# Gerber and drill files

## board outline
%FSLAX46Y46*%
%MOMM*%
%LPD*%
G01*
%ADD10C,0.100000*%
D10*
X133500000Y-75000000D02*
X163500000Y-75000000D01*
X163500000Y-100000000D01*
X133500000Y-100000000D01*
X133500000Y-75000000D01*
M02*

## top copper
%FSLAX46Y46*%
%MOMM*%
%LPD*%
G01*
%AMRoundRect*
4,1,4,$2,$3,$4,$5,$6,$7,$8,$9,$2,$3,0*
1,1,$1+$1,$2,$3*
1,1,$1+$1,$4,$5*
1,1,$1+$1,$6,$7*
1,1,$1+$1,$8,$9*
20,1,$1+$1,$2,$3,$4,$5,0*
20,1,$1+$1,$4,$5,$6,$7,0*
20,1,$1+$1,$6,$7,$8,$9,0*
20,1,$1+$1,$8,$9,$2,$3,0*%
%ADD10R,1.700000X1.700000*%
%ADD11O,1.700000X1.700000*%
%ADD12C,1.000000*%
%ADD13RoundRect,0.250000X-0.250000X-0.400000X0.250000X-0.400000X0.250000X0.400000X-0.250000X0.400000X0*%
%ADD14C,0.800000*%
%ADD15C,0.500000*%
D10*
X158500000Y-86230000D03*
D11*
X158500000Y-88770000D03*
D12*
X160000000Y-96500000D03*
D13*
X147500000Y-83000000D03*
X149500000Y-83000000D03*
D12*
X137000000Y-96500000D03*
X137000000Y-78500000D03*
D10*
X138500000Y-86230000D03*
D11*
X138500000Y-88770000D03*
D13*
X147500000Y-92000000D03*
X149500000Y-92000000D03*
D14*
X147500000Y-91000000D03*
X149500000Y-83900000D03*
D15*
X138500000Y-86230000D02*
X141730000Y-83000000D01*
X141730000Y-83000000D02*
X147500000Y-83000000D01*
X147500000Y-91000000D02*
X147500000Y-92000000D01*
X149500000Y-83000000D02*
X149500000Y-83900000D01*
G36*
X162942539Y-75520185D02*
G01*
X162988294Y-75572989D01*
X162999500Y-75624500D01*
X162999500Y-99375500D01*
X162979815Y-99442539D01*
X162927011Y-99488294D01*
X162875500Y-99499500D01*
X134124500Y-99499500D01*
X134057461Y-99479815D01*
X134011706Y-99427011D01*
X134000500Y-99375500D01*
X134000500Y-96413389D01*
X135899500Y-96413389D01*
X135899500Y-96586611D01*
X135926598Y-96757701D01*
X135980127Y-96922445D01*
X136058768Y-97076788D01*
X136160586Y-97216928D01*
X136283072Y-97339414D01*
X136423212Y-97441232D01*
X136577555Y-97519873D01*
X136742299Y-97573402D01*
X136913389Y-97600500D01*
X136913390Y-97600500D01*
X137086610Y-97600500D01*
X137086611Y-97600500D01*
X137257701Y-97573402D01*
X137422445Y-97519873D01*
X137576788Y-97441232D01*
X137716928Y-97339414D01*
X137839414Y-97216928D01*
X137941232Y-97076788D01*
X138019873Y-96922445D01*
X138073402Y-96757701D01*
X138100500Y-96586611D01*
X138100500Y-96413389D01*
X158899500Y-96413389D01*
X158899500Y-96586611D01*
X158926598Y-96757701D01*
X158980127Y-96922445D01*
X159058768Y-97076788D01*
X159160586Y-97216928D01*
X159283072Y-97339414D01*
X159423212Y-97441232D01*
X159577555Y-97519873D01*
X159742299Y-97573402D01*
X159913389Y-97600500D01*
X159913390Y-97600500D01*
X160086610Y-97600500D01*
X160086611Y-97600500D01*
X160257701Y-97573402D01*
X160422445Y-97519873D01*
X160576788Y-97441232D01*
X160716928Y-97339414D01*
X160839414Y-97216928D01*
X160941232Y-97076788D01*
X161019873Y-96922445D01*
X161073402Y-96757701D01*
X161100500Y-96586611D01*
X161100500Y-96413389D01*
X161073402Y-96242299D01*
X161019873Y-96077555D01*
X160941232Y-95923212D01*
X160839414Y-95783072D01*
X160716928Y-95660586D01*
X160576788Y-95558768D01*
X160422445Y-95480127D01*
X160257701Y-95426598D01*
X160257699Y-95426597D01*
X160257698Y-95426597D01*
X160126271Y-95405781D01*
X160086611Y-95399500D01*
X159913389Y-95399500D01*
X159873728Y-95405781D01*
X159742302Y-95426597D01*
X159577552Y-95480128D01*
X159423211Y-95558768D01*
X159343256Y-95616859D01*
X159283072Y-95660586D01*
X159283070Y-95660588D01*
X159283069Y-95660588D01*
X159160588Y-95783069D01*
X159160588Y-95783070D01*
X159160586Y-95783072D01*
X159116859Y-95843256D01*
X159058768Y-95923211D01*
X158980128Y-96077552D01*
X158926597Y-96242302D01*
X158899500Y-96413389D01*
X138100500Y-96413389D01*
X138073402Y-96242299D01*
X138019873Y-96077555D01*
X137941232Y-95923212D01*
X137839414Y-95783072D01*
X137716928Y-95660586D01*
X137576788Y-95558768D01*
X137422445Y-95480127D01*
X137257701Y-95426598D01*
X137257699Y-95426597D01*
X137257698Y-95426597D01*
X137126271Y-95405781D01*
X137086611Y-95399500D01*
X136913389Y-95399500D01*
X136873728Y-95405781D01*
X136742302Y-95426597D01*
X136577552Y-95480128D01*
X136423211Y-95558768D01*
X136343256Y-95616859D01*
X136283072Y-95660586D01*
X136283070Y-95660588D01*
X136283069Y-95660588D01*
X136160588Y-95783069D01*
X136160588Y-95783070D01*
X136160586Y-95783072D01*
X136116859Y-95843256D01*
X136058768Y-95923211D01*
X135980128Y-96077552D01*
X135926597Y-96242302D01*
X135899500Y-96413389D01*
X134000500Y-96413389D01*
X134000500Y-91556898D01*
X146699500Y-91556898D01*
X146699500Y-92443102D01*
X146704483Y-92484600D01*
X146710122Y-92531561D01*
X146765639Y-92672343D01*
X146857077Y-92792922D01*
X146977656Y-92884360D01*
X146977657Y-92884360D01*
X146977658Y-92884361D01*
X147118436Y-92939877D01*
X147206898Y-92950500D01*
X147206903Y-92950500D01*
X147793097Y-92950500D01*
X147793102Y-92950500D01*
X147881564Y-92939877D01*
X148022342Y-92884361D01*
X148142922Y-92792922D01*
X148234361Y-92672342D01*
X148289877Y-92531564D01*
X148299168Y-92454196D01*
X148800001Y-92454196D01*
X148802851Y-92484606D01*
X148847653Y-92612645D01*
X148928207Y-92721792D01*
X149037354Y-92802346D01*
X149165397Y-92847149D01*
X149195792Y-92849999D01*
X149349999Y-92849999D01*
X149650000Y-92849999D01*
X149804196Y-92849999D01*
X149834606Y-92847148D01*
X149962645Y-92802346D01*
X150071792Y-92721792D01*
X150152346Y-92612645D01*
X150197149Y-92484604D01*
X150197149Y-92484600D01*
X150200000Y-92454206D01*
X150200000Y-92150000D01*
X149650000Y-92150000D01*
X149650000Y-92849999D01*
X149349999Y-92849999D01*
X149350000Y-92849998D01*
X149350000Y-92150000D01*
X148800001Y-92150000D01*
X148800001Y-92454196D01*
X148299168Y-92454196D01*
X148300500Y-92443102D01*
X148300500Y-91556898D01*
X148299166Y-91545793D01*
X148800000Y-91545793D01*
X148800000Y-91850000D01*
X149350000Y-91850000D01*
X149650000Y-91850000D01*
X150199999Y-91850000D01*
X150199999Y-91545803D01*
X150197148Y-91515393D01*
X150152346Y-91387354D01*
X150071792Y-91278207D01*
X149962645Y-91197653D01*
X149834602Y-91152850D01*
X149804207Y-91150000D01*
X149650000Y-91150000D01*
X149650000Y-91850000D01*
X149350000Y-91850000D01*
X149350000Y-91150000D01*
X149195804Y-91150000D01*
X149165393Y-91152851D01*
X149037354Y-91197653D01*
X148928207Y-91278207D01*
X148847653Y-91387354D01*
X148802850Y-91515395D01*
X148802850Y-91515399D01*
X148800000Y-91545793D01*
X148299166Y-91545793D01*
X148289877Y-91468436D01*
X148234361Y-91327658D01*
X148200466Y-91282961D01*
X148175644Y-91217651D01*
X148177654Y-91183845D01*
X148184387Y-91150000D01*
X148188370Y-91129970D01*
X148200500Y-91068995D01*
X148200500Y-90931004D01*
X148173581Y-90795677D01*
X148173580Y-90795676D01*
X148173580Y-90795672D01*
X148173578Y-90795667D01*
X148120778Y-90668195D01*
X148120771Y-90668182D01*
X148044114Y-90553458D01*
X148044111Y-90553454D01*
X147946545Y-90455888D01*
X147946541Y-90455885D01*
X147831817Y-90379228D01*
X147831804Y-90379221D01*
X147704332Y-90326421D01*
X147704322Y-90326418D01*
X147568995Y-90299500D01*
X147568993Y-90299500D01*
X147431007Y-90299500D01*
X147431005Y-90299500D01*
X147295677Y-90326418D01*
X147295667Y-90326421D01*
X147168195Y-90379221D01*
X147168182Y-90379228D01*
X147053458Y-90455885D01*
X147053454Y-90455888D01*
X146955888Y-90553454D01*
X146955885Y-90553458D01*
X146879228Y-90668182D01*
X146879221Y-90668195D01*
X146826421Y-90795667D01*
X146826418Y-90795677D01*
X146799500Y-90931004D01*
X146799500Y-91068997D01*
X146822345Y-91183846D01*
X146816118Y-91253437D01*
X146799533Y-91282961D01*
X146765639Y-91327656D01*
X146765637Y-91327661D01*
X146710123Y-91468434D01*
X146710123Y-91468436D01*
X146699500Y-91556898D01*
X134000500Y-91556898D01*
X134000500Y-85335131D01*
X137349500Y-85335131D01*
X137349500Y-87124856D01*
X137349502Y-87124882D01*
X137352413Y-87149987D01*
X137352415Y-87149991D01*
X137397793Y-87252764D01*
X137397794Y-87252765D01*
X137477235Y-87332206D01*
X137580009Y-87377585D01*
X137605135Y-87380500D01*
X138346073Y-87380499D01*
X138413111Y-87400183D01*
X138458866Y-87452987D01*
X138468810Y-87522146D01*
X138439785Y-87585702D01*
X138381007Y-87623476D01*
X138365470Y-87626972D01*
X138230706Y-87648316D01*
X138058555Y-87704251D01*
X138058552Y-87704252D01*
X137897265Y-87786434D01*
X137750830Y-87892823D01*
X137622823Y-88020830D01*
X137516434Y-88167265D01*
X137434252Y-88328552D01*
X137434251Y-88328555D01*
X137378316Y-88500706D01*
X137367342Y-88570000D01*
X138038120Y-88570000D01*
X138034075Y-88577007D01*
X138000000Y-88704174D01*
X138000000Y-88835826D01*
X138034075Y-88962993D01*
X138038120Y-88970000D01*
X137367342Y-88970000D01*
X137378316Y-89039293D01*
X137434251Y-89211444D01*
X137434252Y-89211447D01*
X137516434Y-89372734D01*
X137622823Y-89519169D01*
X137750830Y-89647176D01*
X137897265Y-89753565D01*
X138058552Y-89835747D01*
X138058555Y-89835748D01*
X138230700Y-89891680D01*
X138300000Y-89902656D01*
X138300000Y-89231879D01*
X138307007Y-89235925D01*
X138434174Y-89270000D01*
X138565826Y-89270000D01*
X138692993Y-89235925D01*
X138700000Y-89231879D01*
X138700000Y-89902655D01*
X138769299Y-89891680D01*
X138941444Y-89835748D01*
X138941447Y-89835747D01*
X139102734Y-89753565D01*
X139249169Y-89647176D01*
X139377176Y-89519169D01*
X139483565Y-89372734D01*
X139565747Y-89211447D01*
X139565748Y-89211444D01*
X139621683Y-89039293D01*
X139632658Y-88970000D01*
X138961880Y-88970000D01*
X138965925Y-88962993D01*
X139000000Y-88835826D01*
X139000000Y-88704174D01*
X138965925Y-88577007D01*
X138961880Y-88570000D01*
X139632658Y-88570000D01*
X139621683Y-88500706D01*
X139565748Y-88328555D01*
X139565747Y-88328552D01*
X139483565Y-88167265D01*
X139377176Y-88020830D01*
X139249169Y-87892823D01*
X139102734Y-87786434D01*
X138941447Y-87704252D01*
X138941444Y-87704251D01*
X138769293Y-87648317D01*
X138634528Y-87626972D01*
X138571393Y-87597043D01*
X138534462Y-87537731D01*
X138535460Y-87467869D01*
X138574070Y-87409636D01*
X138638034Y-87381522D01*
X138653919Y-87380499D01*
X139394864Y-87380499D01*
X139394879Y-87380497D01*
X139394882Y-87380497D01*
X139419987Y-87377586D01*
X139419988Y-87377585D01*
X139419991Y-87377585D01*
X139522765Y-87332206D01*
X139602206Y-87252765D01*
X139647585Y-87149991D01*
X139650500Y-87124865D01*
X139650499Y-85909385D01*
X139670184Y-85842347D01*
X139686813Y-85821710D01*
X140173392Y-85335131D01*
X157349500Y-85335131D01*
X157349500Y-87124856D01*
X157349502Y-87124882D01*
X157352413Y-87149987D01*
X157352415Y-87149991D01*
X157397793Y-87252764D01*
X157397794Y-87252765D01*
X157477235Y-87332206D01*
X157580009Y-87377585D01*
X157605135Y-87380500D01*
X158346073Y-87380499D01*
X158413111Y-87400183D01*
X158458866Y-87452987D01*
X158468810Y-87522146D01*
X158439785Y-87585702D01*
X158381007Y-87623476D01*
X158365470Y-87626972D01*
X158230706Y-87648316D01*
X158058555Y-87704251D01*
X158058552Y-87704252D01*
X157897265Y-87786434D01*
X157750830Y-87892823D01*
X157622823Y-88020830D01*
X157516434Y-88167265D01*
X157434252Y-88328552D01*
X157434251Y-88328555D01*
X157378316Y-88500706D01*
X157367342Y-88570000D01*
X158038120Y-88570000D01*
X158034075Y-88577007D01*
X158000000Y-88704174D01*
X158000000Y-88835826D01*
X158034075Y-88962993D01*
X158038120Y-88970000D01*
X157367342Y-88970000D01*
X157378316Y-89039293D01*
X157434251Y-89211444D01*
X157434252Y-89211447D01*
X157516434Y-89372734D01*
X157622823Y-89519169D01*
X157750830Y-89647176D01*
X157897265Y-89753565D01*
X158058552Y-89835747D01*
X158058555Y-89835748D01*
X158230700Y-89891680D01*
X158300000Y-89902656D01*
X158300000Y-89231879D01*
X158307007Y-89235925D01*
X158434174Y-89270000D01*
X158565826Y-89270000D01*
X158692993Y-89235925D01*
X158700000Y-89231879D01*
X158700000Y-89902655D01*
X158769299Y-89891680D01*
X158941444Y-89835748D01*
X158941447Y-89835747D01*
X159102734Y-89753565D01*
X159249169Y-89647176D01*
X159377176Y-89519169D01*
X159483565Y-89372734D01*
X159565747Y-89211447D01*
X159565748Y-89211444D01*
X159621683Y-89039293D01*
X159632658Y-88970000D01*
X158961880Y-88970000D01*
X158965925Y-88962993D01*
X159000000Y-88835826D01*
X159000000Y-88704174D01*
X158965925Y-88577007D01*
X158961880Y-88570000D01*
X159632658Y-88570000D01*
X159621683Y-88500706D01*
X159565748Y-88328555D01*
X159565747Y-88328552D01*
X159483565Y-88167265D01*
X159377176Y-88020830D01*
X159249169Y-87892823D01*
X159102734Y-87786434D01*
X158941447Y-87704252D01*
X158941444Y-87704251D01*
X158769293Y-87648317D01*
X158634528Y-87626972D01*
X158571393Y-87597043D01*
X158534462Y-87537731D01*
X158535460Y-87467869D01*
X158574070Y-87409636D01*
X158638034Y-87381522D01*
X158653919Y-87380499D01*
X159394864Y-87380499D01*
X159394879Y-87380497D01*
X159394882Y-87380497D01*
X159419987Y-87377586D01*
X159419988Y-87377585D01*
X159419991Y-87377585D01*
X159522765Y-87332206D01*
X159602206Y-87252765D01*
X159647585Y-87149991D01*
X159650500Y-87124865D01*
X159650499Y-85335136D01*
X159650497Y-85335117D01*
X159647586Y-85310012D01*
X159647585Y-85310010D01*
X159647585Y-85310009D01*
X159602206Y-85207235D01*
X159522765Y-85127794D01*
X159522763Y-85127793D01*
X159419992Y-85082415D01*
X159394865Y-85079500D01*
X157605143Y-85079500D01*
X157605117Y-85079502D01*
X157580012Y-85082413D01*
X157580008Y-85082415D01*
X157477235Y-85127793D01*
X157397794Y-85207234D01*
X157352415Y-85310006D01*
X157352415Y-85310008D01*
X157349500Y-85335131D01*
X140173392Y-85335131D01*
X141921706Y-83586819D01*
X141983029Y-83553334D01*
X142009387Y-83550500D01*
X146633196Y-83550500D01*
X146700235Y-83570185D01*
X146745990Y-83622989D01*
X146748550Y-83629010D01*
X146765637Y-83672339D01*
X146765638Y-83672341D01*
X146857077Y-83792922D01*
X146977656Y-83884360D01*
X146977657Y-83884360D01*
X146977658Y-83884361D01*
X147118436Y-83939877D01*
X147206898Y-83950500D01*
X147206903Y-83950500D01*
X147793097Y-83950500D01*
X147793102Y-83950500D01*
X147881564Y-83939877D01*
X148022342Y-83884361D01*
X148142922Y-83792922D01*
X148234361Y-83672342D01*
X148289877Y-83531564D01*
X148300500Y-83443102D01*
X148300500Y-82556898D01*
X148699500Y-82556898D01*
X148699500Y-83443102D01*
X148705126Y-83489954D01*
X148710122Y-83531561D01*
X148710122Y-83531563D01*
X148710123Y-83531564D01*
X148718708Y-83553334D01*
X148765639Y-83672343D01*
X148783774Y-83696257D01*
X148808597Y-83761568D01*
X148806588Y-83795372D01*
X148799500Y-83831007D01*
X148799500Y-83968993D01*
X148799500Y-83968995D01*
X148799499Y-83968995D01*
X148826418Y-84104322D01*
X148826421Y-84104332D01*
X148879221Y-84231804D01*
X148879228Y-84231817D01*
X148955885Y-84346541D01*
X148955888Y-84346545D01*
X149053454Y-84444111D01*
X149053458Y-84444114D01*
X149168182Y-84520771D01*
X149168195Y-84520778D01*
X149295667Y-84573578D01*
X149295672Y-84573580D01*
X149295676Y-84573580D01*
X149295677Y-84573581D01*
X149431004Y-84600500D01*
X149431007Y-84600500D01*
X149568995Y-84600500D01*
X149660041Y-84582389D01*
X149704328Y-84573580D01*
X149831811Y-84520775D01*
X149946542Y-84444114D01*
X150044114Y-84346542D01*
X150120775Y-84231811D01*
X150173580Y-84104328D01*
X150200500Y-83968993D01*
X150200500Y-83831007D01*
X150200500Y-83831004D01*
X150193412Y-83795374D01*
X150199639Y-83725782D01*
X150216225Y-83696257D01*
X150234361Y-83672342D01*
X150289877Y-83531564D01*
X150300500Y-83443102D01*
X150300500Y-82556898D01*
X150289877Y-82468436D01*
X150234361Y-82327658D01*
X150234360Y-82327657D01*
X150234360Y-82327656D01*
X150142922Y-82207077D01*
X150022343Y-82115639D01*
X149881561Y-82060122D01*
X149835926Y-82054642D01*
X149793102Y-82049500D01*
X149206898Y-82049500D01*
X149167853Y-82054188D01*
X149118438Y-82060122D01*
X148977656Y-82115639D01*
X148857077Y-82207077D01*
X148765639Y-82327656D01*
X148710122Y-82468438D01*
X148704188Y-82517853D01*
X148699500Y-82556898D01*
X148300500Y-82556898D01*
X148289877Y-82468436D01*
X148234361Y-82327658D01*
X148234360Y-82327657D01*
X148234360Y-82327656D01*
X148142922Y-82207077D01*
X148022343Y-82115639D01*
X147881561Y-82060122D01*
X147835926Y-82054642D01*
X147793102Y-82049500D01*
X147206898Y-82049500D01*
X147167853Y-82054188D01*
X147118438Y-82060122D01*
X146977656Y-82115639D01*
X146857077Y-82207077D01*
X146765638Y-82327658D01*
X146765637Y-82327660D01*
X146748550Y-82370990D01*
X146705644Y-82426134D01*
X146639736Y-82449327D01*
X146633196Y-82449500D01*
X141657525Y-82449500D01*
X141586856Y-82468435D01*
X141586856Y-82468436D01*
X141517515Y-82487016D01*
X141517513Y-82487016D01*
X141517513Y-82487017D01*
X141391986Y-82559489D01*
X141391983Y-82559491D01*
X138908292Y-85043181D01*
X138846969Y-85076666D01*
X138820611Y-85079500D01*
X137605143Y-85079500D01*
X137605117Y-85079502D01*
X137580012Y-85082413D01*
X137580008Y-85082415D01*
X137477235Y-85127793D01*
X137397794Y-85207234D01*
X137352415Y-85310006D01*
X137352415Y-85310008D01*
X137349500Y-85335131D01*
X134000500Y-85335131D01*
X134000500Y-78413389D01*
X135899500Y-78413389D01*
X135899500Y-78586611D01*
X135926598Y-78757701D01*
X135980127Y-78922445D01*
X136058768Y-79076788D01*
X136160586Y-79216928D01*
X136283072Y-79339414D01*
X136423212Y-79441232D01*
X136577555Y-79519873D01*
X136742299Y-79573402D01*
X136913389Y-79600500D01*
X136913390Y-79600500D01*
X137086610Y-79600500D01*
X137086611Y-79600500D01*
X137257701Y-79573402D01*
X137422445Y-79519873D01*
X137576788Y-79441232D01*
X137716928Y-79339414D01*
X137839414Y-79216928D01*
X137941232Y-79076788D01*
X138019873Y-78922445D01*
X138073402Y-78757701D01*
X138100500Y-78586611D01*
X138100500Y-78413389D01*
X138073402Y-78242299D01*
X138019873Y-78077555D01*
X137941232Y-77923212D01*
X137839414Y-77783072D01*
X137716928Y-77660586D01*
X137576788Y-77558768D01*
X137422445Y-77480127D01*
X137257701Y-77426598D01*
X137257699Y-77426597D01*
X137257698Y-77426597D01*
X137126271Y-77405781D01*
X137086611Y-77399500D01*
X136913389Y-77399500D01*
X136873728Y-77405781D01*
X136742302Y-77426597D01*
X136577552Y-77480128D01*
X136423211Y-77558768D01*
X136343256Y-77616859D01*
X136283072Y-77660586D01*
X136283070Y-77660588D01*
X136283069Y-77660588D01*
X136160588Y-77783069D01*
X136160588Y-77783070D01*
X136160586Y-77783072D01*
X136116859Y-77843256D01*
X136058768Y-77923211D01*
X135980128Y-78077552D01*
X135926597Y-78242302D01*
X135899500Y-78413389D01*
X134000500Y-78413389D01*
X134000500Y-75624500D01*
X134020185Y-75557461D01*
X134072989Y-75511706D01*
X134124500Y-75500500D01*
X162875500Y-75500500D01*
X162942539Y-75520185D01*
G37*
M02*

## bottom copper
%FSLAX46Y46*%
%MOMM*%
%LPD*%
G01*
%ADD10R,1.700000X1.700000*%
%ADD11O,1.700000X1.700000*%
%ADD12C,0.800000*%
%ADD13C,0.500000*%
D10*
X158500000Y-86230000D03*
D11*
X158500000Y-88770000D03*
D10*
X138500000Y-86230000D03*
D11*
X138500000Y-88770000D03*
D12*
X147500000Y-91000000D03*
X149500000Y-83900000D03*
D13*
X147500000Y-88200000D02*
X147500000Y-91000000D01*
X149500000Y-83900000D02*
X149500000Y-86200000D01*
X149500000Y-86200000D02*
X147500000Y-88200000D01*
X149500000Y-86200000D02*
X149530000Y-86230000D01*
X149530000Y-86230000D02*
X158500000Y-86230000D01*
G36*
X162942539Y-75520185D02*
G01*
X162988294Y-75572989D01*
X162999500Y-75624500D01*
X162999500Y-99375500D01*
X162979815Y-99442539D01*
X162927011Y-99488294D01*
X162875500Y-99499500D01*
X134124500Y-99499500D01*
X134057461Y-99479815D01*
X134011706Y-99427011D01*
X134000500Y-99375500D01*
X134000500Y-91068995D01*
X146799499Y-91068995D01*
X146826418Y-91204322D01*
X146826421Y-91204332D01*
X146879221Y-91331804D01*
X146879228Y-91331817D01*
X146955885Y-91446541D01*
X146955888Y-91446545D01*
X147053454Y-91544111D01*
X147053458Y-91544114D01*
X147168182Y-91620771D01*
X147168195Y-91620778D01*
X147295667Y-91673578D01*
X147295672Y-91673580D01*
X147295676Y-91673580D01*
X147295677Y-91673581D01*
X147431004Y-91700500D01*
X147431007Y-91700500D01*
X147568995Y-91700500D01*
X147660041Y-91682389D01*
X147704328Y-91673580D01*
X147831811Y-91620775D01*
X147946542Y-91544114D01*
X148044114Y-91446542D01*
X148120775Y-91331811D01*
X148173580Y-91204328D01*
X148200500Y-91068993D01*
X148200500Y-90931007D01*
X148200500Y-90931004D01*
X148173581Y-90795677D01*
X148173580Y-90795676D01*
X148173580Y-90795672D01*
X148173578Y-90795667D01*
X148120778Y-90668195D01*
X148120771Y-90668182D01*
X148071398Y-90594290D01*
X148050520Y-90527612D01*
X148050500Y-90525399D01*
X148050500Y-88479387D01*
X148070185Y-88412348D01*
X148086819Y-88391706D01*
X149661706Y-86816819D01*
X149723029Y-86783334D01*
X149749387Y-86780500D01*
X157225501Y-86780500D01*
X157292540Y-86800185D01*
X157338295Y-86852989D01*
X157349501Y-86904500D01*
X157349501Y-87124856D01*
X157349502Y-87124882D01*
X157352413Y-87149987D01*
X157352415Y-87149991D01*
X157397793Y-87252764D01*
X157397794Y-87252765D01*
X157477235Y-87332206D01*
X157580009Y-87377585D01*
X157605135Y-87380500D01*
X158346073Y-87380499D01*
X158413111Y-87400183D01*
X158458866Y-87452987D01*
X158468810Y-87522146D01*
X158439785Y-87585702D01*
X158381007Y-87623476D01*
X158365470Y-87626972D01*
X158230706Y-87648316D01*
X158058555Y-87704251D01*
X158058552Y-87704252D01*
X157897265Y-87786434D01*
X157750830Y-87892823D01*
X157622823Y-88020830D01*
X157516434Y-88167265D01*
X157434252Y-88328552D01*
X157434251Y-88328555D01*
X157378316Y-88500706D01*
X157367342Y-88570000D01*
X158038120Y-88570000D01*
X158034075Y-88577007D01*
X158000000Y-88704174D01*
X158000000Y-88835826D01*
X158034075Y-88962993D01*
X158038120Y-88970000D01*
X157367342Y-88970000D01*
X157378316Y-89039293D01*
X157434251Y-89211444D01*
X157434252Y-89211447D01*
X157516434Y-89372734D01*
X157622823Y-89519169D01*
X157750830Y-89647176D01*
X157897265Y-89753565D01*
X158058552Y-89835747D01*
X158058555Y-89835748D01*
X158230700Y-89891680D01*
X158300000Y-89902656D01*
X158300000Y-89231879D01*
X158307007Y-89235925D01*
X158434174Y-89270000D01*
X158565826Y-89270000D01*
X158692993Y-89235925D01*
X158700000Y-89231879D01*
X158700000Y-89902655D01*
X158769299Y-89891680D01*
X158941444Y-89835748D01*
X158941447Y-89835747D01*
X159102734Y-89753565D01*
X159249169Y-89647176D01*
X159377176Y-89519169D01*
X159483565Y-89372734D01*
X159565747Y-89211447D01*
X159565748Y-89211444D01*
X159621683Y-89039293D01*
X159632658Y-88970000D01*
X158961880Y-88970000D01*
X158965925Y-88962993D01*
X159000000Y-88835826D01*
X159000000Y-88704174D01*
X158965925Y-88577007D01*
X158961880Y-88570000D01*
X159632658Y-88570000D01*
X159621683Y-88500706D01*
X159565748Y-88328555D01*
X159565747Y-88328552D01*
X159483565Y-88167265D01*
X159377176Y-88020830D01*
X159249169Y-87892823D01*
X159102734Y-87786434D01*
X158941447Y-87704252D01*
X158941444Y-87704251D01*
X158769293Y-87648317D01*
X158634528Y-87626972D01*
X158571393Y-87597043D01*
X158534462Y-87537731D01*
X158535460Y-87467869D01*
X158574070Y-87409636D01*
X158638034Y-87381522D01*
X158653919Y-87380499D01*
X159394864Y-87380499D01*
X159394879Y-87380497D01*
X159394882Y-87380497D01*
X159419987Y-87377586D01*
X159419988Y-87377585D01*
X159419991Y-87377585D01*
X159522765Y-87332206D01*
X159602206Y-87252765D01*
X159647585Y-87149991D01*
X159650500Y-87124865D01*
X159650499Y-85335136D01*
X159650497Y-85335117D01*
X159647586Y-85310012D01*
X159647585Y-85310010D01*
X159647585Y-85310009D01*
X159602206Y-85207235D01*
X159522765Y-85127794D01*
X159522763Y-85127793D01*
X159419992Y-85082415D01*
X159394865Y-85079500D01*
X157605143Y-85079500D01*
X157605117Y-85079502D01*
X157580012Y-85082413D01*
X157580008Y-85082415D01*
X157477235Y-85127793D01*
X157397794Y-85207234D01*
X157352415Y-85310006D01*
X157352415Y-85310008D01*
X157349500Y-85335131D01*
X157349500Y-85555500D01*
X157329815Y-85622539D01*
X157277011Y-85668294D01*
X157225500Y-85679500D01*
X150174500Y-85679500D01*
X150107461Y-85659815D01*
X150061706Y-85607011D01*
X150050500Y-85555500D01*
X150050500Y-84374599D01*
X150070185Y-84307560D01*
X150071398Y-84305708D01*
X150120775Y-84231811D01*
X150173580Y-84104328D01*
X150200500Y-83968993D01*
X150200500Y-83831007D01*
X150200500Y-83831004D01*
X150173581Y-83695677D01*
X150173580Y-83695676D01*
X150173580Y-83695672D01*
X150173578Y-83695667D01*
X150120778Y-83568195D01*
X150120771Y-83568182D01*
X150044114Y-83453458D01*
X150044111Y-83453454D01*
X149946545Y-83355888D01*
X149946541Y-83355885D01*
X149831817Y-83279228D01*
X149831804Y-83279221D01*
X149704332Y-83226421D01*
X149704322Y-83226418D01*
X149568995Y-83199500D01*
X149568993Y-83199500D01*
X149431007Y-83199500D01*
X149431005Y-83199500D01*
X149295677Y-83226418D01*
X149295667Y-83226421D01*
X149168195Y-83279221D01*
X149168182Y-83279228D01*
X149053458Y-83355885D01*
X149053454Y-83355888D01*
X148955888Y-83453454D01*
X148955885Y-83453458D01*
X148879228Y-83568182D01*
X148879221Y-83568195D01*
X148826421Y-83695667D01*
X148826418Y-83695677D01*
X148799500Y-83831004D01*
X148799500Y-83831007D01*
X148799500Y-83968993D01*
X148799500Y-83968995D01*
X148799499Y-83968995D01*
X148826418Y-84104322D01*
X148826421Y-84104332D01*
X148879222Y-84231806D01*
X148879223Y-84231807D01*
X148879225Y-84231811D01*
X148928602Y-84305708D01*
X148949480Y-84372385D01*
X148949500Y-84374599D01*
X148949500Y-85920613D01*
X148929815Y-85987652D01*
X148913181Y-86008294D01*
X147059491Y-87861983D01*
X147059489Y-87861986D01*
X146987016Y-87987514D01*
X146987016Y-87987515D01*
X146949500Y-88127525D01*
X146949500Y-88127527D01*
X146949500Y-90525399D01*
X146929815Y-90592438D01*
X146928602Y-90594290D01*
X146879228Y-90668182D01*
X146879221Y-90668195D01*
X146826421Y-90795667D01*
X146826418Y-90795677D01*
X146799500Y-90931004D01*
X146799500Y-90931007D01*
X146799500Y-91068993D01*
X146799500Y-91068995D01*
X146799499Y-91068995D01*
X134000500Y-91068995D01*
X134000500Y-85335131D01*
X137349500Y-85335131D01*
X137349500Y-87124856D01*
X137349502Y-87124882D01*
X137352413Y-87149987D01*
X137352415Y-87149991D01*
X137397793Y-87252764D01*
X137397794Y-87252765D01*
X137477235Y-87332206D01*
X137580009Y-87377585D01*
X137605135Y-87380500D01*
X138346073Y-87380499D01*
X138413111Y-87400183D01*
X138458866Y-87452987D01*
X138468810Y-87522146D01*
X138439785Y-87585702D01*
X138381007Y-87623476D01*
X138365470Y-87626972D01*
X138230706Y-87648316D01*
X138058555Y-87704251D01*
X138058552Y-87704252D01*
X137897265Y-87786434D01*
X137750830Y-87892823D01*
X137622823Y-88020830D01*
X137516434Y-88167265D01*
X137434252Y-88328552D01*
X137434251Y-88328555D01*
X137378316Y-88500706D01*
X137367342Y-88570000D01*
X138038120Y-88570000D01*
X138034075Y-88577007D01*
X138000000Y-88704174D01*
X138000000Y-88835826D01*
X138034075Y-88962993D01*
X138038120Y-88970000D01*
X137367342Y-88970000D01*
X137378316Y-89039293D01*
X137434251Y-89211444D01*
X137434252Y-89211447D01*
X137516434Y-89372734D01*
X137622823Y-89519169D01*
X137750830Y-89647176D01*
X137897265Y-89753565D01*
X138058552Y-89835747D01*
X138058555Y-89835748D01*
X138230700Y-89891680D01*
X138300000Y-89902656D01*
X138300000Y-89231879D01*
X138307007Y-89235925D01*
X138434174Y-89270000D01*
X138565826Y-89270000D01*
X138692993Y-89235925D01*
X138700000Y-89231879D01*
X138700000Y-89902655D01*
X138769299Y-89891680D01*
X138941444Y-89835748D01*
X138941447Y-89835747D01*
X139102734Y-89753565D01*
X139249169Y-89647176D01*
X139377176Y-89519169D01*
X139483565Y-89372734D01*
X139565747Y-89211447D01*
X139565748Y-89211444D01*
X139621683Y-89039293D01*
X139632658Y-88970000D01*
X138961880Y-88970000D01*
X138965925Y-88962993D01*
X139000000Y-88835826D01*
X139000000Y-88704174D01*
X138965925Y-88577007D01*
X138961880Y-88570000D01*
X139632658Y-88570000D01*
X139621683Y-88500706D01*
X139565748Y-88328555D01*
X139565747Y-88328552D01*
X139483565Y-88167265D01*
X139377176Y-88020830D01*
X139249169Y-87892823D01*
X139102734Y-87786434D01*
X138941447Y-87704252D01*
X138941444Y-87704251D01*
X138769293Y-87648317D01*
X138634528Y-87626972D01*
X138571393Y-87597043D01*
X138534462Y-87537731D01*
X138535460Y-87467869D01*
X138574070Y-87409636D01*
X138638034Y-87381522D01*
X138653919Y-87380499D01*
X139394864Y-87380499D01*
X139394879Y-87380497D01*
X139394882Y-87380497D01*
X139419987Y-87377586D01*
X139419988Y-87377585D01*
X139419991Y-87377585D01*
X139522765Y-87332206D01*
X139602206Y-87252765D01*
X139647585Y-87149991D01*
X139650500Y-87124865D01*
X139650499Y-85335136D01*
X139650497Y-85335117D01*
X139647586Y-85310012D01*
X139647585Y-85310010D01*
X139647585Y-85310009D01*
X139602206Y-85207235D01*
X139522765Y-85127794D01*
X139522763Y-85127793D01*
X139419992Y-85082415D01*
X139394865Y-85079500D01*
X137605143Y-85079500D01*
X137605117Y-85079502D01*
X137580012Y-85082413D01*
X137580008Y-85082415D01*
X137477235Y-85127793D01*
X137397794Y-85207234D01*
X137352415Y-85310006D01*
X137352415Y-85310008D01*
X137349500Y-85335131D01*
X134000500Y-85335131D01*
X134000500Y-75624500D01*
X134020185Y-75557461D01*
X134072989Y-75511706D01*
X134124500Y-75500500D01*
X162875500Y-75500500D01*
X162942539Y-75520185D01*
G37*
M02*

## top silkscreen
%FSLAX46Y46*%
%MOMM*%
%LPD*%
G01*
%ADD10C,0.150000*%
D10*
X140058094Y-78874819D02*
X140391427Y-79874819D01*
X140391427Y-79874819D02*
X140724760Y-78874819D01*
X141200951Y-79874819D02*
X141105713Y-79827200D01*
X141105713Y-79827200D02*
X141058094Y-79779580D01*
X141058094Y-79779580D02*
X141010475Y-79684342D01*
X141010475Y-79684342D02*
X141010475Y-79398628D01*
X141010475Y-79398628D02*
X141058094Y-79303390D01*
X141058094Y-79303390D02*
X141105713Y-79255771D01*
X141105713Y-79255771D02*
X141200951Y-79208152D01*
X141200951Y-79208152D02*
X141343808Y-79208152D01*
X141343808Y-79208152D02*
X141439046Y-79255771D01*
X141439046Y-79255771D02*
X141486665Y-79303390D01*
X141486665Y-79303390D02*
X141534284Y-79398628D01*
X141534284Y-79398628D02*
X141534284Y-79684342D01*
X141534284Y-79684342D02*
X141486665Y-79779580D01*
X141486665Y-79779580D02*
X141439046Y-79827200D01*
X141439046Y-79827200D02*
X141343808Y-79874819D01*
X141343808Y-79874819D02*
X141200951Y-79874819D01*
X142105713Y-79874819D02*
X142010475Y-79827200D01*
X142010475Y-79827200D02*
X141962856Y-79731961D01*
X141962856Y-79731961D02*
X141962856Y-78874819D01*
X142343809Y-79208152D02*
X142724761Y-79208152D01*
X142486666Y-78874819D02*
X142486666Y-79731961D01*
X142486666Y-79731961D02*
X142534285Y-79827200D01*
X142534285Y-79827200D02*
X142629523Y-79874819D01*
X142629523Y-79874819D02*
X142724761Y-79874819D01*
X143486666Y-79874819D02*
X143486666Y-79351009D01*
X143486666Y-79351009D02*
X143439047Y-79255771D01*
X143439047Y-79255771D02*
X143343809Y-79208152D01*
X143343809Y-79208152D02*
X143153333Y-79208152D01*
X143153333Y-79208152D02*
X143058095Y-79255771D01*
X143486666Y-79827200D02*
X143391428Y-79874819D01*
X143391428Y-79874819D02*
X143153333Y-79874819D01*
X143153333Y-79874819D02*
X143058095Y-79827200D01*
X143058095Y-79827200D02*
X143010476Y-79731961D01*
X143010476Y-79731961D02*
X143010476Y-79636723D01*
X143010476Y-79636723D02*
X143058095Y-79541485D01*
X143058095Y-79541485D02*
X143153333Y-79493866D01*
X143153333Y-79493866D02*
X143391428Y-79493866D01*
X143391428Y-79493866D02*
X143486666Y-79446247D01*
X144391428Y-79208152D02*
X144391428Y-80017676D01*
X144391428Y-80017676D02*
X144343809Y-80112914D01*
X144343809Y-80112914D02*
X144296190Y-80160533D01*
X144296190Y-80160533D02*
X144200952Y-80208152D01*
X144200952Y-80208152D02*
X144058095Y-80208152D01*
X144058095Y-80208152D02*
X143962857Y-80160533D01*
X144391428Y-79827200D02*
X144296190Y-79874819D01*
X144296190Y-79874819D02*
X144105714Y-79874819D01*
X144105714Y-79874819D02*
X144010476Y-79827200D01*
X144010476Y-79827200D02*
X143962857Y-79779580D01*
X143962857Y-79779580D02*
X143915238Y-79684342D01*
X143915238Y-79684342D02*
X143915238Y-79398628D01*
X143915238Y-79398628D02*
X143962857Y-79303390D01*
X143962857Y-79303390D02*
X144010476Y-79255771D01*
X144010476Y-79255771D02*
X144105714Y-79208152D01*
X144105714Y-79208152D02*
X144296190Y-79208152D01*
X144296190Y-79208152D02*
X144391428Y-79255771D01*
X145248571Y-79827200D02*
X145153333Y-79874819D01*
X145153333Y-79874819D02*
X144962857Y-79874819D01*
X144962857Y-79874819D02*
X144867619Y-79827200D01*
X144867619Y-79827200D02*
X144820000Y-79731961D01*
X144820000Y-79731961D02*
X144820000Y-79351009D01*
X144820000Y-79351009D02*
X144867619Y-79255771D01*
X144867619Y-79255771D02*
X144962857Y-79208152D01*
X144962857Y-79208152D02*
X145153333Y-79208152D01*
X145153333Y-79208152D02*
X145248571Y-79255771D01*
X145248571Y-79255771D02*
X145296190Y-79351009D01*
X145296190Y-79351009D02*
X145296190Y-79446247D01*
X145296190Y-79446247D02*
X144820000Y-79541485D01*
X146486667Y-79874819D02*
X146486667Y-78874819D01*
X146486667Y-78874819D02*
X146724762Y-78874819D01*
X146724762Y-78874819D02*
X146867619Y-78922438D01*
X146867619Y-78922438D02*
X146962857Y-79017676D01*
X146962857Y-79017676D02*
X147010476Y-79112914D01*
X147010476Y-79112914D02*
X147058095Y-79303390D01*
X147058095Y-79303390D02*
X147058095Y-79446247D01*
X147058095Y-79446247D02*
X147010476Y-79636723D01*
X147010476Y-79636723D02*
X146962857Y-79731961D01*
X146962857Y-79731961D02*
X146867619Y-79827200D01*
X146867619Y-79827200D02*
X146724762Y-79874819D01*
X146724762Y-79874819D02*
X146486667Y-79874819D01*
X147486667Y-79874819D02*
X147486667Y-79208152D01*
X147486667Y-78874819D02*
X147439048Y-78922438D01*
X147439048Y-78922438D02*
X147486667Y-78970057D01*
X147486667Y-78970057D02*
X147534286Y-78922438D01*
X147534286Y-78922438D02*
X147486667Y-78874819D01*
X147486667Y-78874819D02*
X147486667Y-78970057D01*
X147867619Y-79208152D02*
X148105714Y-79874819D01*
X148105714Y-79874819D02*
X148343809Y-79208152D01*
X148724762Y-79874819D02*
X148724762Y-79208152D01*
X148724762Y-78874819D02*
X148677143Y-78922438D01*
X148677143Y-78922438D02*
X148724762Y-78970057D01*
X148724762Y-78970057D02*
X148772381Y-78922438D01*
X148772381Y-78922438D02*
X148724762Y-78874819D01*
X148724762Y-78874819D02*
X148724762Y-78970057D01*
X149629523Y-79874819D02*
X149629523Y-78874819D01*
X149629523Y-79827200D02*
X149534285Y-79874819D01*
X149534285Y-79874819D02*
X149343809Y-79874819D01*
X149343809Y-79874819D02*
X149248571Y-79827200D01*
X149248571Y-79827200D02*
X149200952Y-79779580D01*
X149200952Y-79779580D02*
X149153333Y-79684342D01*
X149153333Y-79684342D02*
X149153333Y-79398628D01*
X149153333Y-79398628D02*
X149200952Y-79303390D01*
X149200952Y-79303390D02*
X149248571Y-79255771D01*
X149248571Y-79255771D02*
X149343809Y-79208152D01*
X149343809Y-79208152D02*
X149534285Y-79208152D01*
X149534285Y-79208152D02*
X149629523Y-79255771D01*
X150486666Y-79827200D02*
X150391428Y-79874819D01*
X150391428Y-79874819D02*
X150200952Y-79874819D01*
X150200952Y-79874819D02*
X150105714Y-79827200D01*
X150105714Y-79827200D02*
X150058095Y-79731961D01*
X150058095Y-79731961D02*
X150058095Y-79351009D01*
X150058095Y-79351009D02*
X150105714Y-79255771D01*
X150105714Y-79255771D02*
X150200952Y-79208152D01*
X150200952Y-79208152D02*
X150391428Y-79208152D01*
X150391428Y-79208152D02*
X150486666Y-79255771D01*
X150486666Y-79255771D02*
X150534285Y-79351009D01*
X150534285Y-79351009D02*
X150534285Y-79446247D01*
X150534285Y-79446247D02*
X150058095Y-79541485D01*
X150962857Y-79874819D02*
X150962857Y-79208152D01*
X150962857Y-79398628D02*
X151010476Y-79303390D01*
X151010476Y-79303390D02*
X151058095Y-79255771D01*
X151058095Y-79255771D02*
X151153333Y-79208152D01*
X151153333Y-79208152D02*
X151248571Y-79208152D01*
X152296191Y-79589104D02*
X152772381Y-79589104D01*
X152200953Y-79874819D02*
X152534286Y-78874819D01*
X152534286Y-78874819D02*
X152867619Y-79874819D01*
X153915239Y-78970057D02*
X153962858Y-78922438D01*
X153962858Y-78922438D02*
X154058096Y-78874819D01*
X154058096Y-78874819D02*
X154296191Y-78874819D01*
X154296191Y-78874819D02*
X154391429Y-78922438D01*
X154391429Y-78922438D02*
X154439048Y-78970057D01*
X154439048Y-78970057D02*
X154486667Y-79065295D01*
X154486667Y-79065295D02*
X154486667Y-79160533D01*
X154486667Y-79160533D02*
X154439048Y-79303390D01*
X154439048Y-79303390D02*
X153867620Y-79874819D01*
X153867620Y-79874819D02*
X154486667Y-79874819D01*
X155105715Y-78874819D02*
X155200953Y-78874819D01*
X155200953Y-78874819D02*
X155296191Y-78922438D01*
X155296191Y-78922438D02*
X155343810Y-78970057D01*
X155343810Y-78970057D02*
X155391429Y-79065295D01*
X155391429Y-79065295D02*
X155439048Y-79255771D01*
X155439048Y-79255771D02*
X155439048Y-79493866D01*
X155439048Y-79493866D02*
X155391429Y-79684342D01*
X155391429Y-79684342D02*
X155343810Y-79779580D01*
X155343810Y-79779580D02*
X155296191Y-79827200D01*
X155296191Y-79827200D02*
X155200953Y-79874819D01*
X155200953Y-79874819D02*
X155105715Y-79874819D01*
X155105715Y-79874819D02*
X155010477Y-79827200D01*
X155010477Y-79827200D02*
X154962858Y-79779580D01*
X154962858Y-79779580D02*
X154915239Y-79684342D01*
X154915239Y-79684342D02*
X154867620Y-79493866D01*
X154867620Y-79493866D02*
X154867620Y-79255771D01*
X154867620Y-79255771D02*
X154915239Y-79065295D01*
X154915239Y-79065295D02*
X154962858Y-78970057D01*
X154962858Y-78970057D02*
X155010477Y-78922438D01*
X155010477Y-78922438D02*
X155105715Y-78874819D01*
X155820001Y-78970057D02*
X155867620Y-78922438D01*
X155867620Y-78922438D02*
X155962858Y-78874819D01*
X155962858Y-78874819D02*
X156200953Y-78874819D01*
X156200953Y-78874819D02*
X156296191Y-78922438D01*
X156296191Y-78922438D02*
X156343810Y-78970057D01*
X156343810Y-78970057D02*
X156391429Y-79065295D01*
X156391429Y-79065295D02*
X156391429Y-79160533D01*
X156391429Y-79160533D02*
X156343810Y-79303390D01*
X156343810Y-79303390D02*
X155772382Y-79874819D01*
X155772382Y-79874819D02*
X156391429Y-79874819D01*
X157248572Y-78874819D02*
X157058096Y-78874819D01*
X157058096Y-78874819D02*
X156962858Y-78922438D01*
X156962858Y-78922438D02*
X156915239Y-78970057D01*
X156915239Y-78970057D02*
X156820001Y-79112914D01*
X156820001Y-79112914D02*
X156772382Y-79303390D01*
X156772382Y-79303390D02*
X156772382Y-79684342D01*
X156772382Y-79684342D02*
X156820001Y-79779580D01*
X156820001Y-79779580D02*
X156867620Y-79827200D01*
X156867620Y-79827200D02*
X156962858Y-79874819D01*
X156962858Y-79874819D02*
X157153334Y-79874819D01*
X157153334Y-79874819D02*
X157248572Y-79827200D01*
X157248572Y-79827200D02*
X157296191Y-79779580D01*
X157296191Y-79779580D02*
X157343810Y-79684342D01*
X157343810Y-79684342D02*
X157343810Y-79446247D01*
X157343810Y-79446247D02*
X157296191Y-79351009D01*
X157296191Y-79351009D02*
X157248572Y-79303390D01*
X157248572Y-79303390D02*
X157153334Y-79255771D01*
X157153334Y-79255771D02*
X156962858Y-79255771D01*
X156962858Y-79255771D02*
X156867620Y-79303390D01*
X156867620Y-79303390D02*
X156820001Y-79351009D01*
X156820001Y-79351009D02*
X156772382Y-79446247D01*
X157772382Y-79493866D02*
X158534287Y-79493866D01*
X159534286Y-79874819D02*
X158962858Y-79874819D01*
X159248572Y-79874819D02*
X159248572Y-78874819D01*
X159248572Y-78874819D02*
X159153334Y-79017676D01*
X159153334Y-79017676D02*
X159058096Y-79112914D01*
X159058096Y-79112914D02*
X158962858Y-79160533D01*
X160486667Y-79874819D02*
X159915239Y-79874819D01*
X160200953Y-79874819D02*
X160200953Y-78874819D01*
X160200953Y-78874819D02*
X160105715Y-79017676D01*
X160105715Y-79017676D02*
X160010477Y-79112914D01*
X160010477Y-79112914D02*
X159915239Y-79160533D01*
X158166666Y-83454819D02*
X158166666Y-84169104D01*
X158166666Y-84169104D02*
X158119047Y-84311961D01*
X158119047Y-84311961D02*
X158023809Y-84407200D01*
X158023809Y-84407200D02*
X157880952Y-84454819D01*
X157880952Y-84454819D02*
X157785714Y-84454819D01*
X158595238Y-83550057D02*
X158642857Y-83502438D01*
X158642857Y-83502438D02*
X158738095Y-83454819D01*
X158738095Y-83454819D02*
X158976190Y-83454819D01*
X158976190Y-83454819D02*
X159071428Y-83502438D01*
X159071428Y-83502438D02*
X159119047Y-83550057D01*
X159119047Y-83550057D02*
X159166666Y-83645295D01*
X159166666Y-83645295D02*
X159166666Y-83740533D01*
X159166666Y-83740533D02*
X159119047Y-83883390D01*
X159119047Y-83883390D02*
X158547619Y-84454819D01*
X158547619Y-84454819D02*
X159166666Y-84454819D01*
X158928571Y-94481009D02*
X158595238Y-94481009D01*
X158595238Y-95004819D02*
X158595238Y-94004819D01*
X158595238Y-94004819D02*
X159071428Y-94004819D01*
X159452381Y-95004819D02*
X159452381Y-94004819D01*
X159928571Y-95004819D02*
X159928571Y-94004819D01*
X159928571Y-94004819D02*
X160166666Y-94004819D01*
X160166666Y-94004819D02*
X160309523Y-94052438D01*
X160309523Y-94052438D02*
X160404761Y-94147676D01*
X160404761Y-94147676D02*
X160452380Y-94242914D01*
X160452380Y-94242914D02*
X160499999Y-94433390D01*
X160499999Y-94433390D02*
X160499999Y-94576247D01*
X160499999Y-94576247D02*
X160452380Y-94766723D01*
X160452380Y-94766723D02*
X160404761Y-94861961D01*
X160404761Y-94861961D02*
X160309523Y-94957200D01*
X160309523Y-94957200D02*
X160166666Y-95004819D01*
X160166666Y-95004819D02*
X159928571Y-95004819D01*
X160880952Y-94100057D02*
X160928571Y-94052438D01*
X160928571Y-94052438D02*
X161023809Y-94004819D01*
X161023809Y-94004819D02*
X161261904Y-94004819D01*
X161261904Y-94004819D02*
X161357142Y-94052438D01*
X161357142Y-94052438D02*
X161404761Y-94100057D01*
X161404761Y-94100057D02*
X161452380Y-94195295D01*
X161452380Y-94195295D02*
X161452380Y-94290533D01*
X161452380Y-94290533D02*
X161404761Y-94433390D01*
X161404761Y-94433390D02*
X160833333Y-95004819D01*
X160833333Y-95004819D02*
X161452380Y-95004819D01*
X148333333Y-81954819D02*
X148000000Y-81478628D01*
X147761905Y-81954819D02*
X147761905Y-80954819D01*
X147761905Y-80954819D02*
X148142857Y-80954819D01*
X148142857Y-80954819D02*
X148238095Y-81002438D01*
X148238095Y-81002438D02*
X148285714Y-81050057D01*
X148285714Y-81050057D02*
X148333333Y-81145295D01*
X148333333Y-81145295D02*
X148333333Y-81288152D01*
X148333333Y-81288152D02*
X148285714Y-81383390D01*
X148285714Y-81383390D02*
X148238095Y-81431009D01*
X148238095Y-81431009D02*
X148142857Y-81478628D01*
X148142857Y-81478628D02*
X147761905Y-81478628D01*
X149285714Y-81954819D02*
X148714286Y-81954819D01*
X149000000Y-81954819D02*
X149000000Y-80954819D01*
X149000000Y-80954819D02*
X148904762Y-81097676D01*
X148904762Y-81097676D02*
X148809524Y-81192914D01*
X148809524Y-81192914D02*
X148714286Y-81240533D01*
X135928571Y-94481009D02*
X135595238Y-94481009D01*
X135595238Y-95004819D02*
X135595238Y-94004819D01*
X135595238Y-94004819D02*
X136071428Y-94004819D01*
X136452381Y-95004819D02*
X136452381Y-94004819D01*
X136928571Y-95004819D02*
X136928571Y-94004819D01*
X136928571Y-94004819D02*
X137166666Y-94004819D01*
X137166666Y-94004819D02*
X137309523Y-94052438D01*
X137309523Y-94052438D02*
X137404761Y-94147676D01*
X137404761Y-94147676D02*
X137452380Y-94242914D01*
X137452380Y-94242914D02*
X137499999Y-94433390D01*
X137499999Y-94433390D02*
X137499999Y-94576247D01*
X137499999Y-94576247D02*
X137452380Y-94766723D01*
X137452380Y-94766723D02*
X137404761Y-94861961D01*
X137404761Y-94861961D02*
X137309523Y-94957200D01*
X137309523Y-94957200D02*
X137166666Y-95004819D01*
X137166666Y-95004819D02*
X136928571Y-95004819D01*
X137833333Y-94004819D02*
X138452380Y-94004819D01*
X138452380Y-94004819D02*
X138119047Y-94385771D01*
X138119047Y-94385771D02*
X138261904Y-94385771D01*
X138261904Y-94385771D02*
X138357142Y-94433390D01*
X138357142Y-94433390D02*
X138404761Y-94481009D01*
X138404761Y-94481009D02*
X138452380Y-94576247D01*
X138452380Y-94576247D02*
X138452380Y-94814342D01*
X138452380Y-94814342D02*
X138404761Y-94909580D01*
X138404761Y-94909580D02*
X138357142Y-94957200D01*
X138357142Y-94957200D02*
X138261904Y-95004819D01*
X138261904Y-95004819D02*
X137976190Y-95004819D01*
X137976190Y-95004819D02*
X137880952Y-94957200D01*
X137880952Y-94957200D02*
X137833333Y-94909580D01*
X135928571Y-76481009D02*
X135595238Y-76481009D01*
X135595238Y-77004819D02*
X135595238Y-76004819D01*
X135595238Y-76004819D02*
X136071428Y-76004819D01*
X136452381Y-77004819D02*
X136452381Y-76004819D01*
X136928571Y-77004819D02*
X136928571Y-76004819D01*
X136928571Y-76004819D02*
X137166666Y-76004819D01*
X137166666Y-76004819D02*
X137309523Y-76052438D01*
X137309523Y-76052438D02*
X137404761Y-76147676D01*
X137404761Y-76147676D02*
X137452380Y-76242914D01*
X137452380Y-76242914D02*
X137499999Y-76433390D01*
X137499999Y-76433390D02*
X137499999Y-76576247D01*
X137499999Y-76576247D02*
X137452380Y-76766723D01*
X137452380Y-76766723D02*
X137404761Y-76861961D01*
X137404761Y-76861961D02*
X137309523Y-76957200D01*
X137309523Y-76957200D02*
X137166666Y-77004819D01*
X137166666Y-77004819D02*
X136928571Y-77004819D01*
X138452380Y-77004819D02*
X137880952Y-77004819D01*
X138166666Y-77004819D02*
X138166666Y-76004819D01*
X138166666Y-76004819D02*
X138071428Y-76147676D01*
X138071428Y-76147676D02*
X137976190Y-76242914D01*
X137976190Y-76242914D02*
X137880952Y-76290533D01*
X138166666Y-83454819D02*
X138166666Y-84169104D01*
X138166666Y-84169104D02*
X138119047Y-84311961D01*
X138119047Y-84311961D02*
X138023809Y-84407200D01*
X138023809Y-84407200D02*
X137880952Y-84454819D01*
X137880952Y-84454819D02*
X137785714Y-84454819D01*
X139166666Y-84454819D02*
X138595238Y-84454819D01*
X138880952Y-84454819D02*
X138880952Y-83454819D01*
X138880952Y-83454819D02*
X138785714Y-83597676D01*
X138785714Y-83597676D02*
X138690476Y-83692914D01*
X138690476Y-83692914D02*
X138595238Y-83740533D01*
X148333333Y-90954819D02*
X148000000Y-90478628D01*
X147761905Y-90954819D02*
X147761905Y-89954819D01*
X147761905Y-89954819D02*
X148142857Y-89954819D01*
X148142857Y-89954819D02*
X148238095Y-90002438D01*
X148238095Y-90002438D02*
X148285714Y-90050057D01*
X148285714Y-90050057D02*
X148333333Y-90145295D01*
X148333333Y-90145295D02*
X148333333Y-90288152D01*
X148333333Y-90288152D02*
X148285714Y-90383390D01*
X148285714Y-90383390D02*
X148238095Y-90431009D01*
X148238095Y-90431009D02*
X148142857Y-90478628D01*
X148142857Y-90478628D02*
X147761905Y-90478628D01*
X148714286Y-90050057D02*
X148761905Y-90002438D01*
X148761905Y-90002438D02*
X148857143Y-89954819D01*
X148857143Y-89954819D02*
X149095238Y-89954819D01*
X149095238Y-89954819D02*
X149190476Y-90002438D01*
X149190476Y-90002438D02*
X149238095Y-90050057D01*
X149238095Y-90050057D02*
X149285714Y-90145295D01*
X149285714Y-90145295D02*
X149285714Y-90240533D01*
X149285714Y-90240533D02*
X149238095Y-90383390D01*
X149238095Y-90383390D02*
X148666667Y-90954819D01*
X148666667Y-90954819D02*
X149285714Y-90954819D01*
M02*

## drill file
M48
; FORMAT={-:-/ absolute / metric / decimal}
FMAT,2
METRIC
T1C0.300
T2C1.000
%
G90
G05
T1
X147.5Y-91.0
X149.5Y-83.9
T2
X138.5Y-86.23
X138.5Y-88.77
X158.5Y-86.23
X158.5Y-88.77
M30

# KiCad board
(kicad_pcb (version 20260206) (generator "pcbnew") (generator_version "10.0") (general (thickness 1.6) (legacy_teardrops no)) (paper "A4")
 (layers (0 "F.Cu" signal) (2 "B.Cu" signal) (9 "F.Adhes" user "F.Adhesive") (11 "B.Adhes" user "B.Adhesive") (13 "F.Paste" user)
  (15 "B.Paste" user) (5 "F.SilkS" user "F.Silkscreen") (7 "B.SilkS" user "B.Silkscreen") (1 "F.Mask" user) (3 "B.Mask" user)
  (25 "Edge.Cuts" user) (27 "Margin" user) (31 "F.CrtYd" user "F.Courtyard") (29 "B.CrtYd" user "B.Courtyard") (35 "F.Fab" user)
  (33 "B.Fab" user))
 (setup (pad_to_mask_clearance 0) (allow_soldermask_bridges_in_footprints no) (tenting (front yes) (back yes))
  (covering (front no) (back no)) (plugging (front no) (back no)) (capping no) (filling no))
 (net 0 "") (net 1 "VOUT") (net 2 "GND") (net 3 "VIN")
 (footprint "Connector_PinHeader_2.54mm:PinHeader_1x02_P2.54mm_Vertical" (layer "F.Cu") (at 158.5 87.5)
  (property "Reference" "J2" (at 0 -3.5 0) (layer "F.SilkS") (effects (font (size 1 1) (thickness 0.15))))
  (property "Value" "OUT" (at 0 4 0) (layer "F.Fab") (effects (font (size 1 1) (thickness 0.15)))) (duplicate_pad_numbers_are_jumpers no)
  (pad "1" thru_hole rect (at 0 -1.27) (size 1.7 1.7) (drill 1) (layers "*.Cu" "*.Mask") (remove_unused_layers no) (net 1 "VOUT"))
  (pad "2" thru_hole oval (at 0 1.27) (size 1.7 1.7) (drill 1) (layers "*.Cu" "*.Mask") (remove_unused_layers no) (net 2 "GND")))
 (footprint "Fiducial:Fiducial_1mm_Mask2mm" (layer "F.Cu") (at 160 96.5)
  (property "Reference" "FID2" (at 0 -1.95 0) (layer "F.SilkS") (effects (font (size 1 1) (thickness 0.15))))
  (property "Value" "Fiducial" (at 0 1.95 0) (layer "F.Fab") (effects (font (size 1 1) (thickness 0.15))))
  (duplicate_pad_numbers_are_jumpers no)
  (pad "" smd circle (at 0 0) (size 1 1) (layers "F.Cu" "F.Mask") (solder_mask_margin 0.5) (clearance 0.6)))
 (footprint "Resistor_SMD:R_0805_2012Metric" (layer "F.Cu") (at 148.5 83)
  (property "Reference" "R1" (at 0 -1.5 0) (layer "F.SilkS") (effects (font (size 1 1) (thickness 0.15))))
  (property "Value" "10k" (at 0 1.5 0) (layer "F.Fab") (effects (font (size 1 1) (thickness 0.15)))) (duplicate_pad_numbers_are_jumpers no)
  (pad "1" smd roundrect (at -1 0) (size 1 1.3) (layers "F.Cu" "F.Mask" "F.Paste") (roundrect_rratio 0.25) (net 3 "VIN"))
  (pad "2" smd roundrect (at 1 0) (size 1 1.3) (layers "F.Cu" "F.Mask" "F.Paste") (roundrect_rratio 0.25) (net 1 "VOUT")))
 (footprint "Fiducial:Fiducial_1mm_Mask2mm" (layer "F.Cu") (at 137 96.5)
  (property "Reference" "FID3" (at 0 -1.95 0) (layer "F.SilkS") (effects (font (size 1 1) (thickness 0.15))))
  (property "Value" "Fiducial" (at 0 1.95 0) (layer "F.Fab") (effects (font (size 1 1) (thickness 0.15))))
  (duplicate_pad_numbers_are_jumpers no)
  (pad "" smd circle (at 0 0) (size 1 1) (layers "F.Cu" "F.Mask") (solder_mask_margin 0.5) (clearance 0.6)))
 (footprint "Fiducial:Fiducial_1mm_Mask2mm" (layer "F.Cu") (at 137 78.5)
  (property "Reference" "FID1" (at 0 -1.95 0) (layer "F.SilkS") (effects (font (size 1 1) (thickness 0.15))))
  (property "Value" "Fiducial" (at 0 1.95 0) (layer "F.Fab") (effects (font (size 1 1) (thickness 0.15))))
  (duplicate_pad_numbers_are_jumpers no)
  (pad "" smd circle (at 0 0) (size 1 1) (layers "F.Cu" "F.Mask") (solder_mask_margin 0.5) (clearance 0.6)))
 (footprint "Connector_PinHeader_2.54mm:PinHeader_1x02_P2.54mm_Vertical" (layer "F.Cu") (at 138.5 87.5)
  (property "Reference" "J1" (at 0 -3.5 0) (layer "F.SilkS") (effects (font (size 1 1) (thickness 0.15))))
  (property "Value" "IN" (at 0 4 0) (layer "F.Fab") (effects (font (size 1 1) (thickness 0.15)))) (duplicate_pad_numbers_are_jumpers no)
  (pad "1" thru_hole rect (at 0 -1.27) (size 1.7 1.7) (drill 1) (layers "*.Cu" "*.Mask") (remove_unused_layers no) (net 3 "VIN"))
  (pad "2" thru_hole oval (at 0 1.27) (size 1.7 1.7) (drill 1) (layers "*.Cu" "*.Mask") (remove_unused_layers no) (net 2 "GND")))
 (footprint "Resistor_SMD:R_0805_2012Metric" (layer "F.Cu") (at 148.5 92)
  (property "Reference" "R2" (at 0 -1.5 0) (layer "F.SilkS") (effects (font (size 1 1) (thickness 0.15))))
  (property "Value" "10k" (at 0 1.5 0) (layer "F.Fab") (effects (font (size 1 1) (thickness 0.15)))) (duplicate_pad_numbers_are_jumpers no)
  (pad "1" smd roundrect (at -1 0) (size 1 1.3) (layers "F.Cu" "F.Mask" "F.Paste") (roundrect_rratio 0.25) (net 1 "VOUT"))
  (pad "2" smd roundrect (at 1 0) (size 1 1.3) (layers "F.Cu" "F.Mask" "F.Paste") (roundrect_rratio 0.25) (thermal_bridge_width 0.3)
   (thermal_gap 0.2) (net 2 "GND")))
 (gr_rect (start 133.5 75) (end 163.5 100) (stroke (width 0.1) (type default)) (fill no) (layer "Edge.Cuts"))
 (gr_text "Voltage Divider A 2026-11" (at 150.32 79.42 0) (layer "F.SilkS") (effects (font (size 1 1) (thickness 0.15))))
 (segment (start 138.5 86.23) (end 141.73 83) (width 0.5) (layer "F.Cu") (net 3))
 (segment (start 141.73 83) (end 147.5 83) (width 0.5) (layer "F.Cu") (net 3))
 (segment (start 147.5 91) (end 147.5 92) (width 0.5) (layer "F.Cu") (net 1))
 (segment (start 149.5 83) (end 149.5 83.9) (width 0.5) (layer "F.Cu") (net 1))
 (via (at 147.5 91) (size 0.8) (drill 0.3) (layers "F.Cu" "B.Cu") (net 1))
 (via (at 149.5 83.9) (size 0.8) (drill 0.3) (layers "F.Cu" "B.Cu") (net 1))
 (segment (start 147.5 88.2) (end 147.5 91) (width 0.5) (layer "B.Cu") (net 1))
 (segment (start 149.5 83.9) (end 149.5 86.2) (width 0.5) (layer "B.Cu") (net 1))
 (segment (start 149.5 86.2) (end 147.5 88.2) (width 0.5) (layer "B.Cu") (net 1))
 (segment (start 149.5 86.2) (end 149.53 86.23) (width 0.5) (layer "B.Cu") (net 1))
 (segment (start 149.53 86.23) (end 158.5 86.23) (width 0.5) (layer "B.Cu") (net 1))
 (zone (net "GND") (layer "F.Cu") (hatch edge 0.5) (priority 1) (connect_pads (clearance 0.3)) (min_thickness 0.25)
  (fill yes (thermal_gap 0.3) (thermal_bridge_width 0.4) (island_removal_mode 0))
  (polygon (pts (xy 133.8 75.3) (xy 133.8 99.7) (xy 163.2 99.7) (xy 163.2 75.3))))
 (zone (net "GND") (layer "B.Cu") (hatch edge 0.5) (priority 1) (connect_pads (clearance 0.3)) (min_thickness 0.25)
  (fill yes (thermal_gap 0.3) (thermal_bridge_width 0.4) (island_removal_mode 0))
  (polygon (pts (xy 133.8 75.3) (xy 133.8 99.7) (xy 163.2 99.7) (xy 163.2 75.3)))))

